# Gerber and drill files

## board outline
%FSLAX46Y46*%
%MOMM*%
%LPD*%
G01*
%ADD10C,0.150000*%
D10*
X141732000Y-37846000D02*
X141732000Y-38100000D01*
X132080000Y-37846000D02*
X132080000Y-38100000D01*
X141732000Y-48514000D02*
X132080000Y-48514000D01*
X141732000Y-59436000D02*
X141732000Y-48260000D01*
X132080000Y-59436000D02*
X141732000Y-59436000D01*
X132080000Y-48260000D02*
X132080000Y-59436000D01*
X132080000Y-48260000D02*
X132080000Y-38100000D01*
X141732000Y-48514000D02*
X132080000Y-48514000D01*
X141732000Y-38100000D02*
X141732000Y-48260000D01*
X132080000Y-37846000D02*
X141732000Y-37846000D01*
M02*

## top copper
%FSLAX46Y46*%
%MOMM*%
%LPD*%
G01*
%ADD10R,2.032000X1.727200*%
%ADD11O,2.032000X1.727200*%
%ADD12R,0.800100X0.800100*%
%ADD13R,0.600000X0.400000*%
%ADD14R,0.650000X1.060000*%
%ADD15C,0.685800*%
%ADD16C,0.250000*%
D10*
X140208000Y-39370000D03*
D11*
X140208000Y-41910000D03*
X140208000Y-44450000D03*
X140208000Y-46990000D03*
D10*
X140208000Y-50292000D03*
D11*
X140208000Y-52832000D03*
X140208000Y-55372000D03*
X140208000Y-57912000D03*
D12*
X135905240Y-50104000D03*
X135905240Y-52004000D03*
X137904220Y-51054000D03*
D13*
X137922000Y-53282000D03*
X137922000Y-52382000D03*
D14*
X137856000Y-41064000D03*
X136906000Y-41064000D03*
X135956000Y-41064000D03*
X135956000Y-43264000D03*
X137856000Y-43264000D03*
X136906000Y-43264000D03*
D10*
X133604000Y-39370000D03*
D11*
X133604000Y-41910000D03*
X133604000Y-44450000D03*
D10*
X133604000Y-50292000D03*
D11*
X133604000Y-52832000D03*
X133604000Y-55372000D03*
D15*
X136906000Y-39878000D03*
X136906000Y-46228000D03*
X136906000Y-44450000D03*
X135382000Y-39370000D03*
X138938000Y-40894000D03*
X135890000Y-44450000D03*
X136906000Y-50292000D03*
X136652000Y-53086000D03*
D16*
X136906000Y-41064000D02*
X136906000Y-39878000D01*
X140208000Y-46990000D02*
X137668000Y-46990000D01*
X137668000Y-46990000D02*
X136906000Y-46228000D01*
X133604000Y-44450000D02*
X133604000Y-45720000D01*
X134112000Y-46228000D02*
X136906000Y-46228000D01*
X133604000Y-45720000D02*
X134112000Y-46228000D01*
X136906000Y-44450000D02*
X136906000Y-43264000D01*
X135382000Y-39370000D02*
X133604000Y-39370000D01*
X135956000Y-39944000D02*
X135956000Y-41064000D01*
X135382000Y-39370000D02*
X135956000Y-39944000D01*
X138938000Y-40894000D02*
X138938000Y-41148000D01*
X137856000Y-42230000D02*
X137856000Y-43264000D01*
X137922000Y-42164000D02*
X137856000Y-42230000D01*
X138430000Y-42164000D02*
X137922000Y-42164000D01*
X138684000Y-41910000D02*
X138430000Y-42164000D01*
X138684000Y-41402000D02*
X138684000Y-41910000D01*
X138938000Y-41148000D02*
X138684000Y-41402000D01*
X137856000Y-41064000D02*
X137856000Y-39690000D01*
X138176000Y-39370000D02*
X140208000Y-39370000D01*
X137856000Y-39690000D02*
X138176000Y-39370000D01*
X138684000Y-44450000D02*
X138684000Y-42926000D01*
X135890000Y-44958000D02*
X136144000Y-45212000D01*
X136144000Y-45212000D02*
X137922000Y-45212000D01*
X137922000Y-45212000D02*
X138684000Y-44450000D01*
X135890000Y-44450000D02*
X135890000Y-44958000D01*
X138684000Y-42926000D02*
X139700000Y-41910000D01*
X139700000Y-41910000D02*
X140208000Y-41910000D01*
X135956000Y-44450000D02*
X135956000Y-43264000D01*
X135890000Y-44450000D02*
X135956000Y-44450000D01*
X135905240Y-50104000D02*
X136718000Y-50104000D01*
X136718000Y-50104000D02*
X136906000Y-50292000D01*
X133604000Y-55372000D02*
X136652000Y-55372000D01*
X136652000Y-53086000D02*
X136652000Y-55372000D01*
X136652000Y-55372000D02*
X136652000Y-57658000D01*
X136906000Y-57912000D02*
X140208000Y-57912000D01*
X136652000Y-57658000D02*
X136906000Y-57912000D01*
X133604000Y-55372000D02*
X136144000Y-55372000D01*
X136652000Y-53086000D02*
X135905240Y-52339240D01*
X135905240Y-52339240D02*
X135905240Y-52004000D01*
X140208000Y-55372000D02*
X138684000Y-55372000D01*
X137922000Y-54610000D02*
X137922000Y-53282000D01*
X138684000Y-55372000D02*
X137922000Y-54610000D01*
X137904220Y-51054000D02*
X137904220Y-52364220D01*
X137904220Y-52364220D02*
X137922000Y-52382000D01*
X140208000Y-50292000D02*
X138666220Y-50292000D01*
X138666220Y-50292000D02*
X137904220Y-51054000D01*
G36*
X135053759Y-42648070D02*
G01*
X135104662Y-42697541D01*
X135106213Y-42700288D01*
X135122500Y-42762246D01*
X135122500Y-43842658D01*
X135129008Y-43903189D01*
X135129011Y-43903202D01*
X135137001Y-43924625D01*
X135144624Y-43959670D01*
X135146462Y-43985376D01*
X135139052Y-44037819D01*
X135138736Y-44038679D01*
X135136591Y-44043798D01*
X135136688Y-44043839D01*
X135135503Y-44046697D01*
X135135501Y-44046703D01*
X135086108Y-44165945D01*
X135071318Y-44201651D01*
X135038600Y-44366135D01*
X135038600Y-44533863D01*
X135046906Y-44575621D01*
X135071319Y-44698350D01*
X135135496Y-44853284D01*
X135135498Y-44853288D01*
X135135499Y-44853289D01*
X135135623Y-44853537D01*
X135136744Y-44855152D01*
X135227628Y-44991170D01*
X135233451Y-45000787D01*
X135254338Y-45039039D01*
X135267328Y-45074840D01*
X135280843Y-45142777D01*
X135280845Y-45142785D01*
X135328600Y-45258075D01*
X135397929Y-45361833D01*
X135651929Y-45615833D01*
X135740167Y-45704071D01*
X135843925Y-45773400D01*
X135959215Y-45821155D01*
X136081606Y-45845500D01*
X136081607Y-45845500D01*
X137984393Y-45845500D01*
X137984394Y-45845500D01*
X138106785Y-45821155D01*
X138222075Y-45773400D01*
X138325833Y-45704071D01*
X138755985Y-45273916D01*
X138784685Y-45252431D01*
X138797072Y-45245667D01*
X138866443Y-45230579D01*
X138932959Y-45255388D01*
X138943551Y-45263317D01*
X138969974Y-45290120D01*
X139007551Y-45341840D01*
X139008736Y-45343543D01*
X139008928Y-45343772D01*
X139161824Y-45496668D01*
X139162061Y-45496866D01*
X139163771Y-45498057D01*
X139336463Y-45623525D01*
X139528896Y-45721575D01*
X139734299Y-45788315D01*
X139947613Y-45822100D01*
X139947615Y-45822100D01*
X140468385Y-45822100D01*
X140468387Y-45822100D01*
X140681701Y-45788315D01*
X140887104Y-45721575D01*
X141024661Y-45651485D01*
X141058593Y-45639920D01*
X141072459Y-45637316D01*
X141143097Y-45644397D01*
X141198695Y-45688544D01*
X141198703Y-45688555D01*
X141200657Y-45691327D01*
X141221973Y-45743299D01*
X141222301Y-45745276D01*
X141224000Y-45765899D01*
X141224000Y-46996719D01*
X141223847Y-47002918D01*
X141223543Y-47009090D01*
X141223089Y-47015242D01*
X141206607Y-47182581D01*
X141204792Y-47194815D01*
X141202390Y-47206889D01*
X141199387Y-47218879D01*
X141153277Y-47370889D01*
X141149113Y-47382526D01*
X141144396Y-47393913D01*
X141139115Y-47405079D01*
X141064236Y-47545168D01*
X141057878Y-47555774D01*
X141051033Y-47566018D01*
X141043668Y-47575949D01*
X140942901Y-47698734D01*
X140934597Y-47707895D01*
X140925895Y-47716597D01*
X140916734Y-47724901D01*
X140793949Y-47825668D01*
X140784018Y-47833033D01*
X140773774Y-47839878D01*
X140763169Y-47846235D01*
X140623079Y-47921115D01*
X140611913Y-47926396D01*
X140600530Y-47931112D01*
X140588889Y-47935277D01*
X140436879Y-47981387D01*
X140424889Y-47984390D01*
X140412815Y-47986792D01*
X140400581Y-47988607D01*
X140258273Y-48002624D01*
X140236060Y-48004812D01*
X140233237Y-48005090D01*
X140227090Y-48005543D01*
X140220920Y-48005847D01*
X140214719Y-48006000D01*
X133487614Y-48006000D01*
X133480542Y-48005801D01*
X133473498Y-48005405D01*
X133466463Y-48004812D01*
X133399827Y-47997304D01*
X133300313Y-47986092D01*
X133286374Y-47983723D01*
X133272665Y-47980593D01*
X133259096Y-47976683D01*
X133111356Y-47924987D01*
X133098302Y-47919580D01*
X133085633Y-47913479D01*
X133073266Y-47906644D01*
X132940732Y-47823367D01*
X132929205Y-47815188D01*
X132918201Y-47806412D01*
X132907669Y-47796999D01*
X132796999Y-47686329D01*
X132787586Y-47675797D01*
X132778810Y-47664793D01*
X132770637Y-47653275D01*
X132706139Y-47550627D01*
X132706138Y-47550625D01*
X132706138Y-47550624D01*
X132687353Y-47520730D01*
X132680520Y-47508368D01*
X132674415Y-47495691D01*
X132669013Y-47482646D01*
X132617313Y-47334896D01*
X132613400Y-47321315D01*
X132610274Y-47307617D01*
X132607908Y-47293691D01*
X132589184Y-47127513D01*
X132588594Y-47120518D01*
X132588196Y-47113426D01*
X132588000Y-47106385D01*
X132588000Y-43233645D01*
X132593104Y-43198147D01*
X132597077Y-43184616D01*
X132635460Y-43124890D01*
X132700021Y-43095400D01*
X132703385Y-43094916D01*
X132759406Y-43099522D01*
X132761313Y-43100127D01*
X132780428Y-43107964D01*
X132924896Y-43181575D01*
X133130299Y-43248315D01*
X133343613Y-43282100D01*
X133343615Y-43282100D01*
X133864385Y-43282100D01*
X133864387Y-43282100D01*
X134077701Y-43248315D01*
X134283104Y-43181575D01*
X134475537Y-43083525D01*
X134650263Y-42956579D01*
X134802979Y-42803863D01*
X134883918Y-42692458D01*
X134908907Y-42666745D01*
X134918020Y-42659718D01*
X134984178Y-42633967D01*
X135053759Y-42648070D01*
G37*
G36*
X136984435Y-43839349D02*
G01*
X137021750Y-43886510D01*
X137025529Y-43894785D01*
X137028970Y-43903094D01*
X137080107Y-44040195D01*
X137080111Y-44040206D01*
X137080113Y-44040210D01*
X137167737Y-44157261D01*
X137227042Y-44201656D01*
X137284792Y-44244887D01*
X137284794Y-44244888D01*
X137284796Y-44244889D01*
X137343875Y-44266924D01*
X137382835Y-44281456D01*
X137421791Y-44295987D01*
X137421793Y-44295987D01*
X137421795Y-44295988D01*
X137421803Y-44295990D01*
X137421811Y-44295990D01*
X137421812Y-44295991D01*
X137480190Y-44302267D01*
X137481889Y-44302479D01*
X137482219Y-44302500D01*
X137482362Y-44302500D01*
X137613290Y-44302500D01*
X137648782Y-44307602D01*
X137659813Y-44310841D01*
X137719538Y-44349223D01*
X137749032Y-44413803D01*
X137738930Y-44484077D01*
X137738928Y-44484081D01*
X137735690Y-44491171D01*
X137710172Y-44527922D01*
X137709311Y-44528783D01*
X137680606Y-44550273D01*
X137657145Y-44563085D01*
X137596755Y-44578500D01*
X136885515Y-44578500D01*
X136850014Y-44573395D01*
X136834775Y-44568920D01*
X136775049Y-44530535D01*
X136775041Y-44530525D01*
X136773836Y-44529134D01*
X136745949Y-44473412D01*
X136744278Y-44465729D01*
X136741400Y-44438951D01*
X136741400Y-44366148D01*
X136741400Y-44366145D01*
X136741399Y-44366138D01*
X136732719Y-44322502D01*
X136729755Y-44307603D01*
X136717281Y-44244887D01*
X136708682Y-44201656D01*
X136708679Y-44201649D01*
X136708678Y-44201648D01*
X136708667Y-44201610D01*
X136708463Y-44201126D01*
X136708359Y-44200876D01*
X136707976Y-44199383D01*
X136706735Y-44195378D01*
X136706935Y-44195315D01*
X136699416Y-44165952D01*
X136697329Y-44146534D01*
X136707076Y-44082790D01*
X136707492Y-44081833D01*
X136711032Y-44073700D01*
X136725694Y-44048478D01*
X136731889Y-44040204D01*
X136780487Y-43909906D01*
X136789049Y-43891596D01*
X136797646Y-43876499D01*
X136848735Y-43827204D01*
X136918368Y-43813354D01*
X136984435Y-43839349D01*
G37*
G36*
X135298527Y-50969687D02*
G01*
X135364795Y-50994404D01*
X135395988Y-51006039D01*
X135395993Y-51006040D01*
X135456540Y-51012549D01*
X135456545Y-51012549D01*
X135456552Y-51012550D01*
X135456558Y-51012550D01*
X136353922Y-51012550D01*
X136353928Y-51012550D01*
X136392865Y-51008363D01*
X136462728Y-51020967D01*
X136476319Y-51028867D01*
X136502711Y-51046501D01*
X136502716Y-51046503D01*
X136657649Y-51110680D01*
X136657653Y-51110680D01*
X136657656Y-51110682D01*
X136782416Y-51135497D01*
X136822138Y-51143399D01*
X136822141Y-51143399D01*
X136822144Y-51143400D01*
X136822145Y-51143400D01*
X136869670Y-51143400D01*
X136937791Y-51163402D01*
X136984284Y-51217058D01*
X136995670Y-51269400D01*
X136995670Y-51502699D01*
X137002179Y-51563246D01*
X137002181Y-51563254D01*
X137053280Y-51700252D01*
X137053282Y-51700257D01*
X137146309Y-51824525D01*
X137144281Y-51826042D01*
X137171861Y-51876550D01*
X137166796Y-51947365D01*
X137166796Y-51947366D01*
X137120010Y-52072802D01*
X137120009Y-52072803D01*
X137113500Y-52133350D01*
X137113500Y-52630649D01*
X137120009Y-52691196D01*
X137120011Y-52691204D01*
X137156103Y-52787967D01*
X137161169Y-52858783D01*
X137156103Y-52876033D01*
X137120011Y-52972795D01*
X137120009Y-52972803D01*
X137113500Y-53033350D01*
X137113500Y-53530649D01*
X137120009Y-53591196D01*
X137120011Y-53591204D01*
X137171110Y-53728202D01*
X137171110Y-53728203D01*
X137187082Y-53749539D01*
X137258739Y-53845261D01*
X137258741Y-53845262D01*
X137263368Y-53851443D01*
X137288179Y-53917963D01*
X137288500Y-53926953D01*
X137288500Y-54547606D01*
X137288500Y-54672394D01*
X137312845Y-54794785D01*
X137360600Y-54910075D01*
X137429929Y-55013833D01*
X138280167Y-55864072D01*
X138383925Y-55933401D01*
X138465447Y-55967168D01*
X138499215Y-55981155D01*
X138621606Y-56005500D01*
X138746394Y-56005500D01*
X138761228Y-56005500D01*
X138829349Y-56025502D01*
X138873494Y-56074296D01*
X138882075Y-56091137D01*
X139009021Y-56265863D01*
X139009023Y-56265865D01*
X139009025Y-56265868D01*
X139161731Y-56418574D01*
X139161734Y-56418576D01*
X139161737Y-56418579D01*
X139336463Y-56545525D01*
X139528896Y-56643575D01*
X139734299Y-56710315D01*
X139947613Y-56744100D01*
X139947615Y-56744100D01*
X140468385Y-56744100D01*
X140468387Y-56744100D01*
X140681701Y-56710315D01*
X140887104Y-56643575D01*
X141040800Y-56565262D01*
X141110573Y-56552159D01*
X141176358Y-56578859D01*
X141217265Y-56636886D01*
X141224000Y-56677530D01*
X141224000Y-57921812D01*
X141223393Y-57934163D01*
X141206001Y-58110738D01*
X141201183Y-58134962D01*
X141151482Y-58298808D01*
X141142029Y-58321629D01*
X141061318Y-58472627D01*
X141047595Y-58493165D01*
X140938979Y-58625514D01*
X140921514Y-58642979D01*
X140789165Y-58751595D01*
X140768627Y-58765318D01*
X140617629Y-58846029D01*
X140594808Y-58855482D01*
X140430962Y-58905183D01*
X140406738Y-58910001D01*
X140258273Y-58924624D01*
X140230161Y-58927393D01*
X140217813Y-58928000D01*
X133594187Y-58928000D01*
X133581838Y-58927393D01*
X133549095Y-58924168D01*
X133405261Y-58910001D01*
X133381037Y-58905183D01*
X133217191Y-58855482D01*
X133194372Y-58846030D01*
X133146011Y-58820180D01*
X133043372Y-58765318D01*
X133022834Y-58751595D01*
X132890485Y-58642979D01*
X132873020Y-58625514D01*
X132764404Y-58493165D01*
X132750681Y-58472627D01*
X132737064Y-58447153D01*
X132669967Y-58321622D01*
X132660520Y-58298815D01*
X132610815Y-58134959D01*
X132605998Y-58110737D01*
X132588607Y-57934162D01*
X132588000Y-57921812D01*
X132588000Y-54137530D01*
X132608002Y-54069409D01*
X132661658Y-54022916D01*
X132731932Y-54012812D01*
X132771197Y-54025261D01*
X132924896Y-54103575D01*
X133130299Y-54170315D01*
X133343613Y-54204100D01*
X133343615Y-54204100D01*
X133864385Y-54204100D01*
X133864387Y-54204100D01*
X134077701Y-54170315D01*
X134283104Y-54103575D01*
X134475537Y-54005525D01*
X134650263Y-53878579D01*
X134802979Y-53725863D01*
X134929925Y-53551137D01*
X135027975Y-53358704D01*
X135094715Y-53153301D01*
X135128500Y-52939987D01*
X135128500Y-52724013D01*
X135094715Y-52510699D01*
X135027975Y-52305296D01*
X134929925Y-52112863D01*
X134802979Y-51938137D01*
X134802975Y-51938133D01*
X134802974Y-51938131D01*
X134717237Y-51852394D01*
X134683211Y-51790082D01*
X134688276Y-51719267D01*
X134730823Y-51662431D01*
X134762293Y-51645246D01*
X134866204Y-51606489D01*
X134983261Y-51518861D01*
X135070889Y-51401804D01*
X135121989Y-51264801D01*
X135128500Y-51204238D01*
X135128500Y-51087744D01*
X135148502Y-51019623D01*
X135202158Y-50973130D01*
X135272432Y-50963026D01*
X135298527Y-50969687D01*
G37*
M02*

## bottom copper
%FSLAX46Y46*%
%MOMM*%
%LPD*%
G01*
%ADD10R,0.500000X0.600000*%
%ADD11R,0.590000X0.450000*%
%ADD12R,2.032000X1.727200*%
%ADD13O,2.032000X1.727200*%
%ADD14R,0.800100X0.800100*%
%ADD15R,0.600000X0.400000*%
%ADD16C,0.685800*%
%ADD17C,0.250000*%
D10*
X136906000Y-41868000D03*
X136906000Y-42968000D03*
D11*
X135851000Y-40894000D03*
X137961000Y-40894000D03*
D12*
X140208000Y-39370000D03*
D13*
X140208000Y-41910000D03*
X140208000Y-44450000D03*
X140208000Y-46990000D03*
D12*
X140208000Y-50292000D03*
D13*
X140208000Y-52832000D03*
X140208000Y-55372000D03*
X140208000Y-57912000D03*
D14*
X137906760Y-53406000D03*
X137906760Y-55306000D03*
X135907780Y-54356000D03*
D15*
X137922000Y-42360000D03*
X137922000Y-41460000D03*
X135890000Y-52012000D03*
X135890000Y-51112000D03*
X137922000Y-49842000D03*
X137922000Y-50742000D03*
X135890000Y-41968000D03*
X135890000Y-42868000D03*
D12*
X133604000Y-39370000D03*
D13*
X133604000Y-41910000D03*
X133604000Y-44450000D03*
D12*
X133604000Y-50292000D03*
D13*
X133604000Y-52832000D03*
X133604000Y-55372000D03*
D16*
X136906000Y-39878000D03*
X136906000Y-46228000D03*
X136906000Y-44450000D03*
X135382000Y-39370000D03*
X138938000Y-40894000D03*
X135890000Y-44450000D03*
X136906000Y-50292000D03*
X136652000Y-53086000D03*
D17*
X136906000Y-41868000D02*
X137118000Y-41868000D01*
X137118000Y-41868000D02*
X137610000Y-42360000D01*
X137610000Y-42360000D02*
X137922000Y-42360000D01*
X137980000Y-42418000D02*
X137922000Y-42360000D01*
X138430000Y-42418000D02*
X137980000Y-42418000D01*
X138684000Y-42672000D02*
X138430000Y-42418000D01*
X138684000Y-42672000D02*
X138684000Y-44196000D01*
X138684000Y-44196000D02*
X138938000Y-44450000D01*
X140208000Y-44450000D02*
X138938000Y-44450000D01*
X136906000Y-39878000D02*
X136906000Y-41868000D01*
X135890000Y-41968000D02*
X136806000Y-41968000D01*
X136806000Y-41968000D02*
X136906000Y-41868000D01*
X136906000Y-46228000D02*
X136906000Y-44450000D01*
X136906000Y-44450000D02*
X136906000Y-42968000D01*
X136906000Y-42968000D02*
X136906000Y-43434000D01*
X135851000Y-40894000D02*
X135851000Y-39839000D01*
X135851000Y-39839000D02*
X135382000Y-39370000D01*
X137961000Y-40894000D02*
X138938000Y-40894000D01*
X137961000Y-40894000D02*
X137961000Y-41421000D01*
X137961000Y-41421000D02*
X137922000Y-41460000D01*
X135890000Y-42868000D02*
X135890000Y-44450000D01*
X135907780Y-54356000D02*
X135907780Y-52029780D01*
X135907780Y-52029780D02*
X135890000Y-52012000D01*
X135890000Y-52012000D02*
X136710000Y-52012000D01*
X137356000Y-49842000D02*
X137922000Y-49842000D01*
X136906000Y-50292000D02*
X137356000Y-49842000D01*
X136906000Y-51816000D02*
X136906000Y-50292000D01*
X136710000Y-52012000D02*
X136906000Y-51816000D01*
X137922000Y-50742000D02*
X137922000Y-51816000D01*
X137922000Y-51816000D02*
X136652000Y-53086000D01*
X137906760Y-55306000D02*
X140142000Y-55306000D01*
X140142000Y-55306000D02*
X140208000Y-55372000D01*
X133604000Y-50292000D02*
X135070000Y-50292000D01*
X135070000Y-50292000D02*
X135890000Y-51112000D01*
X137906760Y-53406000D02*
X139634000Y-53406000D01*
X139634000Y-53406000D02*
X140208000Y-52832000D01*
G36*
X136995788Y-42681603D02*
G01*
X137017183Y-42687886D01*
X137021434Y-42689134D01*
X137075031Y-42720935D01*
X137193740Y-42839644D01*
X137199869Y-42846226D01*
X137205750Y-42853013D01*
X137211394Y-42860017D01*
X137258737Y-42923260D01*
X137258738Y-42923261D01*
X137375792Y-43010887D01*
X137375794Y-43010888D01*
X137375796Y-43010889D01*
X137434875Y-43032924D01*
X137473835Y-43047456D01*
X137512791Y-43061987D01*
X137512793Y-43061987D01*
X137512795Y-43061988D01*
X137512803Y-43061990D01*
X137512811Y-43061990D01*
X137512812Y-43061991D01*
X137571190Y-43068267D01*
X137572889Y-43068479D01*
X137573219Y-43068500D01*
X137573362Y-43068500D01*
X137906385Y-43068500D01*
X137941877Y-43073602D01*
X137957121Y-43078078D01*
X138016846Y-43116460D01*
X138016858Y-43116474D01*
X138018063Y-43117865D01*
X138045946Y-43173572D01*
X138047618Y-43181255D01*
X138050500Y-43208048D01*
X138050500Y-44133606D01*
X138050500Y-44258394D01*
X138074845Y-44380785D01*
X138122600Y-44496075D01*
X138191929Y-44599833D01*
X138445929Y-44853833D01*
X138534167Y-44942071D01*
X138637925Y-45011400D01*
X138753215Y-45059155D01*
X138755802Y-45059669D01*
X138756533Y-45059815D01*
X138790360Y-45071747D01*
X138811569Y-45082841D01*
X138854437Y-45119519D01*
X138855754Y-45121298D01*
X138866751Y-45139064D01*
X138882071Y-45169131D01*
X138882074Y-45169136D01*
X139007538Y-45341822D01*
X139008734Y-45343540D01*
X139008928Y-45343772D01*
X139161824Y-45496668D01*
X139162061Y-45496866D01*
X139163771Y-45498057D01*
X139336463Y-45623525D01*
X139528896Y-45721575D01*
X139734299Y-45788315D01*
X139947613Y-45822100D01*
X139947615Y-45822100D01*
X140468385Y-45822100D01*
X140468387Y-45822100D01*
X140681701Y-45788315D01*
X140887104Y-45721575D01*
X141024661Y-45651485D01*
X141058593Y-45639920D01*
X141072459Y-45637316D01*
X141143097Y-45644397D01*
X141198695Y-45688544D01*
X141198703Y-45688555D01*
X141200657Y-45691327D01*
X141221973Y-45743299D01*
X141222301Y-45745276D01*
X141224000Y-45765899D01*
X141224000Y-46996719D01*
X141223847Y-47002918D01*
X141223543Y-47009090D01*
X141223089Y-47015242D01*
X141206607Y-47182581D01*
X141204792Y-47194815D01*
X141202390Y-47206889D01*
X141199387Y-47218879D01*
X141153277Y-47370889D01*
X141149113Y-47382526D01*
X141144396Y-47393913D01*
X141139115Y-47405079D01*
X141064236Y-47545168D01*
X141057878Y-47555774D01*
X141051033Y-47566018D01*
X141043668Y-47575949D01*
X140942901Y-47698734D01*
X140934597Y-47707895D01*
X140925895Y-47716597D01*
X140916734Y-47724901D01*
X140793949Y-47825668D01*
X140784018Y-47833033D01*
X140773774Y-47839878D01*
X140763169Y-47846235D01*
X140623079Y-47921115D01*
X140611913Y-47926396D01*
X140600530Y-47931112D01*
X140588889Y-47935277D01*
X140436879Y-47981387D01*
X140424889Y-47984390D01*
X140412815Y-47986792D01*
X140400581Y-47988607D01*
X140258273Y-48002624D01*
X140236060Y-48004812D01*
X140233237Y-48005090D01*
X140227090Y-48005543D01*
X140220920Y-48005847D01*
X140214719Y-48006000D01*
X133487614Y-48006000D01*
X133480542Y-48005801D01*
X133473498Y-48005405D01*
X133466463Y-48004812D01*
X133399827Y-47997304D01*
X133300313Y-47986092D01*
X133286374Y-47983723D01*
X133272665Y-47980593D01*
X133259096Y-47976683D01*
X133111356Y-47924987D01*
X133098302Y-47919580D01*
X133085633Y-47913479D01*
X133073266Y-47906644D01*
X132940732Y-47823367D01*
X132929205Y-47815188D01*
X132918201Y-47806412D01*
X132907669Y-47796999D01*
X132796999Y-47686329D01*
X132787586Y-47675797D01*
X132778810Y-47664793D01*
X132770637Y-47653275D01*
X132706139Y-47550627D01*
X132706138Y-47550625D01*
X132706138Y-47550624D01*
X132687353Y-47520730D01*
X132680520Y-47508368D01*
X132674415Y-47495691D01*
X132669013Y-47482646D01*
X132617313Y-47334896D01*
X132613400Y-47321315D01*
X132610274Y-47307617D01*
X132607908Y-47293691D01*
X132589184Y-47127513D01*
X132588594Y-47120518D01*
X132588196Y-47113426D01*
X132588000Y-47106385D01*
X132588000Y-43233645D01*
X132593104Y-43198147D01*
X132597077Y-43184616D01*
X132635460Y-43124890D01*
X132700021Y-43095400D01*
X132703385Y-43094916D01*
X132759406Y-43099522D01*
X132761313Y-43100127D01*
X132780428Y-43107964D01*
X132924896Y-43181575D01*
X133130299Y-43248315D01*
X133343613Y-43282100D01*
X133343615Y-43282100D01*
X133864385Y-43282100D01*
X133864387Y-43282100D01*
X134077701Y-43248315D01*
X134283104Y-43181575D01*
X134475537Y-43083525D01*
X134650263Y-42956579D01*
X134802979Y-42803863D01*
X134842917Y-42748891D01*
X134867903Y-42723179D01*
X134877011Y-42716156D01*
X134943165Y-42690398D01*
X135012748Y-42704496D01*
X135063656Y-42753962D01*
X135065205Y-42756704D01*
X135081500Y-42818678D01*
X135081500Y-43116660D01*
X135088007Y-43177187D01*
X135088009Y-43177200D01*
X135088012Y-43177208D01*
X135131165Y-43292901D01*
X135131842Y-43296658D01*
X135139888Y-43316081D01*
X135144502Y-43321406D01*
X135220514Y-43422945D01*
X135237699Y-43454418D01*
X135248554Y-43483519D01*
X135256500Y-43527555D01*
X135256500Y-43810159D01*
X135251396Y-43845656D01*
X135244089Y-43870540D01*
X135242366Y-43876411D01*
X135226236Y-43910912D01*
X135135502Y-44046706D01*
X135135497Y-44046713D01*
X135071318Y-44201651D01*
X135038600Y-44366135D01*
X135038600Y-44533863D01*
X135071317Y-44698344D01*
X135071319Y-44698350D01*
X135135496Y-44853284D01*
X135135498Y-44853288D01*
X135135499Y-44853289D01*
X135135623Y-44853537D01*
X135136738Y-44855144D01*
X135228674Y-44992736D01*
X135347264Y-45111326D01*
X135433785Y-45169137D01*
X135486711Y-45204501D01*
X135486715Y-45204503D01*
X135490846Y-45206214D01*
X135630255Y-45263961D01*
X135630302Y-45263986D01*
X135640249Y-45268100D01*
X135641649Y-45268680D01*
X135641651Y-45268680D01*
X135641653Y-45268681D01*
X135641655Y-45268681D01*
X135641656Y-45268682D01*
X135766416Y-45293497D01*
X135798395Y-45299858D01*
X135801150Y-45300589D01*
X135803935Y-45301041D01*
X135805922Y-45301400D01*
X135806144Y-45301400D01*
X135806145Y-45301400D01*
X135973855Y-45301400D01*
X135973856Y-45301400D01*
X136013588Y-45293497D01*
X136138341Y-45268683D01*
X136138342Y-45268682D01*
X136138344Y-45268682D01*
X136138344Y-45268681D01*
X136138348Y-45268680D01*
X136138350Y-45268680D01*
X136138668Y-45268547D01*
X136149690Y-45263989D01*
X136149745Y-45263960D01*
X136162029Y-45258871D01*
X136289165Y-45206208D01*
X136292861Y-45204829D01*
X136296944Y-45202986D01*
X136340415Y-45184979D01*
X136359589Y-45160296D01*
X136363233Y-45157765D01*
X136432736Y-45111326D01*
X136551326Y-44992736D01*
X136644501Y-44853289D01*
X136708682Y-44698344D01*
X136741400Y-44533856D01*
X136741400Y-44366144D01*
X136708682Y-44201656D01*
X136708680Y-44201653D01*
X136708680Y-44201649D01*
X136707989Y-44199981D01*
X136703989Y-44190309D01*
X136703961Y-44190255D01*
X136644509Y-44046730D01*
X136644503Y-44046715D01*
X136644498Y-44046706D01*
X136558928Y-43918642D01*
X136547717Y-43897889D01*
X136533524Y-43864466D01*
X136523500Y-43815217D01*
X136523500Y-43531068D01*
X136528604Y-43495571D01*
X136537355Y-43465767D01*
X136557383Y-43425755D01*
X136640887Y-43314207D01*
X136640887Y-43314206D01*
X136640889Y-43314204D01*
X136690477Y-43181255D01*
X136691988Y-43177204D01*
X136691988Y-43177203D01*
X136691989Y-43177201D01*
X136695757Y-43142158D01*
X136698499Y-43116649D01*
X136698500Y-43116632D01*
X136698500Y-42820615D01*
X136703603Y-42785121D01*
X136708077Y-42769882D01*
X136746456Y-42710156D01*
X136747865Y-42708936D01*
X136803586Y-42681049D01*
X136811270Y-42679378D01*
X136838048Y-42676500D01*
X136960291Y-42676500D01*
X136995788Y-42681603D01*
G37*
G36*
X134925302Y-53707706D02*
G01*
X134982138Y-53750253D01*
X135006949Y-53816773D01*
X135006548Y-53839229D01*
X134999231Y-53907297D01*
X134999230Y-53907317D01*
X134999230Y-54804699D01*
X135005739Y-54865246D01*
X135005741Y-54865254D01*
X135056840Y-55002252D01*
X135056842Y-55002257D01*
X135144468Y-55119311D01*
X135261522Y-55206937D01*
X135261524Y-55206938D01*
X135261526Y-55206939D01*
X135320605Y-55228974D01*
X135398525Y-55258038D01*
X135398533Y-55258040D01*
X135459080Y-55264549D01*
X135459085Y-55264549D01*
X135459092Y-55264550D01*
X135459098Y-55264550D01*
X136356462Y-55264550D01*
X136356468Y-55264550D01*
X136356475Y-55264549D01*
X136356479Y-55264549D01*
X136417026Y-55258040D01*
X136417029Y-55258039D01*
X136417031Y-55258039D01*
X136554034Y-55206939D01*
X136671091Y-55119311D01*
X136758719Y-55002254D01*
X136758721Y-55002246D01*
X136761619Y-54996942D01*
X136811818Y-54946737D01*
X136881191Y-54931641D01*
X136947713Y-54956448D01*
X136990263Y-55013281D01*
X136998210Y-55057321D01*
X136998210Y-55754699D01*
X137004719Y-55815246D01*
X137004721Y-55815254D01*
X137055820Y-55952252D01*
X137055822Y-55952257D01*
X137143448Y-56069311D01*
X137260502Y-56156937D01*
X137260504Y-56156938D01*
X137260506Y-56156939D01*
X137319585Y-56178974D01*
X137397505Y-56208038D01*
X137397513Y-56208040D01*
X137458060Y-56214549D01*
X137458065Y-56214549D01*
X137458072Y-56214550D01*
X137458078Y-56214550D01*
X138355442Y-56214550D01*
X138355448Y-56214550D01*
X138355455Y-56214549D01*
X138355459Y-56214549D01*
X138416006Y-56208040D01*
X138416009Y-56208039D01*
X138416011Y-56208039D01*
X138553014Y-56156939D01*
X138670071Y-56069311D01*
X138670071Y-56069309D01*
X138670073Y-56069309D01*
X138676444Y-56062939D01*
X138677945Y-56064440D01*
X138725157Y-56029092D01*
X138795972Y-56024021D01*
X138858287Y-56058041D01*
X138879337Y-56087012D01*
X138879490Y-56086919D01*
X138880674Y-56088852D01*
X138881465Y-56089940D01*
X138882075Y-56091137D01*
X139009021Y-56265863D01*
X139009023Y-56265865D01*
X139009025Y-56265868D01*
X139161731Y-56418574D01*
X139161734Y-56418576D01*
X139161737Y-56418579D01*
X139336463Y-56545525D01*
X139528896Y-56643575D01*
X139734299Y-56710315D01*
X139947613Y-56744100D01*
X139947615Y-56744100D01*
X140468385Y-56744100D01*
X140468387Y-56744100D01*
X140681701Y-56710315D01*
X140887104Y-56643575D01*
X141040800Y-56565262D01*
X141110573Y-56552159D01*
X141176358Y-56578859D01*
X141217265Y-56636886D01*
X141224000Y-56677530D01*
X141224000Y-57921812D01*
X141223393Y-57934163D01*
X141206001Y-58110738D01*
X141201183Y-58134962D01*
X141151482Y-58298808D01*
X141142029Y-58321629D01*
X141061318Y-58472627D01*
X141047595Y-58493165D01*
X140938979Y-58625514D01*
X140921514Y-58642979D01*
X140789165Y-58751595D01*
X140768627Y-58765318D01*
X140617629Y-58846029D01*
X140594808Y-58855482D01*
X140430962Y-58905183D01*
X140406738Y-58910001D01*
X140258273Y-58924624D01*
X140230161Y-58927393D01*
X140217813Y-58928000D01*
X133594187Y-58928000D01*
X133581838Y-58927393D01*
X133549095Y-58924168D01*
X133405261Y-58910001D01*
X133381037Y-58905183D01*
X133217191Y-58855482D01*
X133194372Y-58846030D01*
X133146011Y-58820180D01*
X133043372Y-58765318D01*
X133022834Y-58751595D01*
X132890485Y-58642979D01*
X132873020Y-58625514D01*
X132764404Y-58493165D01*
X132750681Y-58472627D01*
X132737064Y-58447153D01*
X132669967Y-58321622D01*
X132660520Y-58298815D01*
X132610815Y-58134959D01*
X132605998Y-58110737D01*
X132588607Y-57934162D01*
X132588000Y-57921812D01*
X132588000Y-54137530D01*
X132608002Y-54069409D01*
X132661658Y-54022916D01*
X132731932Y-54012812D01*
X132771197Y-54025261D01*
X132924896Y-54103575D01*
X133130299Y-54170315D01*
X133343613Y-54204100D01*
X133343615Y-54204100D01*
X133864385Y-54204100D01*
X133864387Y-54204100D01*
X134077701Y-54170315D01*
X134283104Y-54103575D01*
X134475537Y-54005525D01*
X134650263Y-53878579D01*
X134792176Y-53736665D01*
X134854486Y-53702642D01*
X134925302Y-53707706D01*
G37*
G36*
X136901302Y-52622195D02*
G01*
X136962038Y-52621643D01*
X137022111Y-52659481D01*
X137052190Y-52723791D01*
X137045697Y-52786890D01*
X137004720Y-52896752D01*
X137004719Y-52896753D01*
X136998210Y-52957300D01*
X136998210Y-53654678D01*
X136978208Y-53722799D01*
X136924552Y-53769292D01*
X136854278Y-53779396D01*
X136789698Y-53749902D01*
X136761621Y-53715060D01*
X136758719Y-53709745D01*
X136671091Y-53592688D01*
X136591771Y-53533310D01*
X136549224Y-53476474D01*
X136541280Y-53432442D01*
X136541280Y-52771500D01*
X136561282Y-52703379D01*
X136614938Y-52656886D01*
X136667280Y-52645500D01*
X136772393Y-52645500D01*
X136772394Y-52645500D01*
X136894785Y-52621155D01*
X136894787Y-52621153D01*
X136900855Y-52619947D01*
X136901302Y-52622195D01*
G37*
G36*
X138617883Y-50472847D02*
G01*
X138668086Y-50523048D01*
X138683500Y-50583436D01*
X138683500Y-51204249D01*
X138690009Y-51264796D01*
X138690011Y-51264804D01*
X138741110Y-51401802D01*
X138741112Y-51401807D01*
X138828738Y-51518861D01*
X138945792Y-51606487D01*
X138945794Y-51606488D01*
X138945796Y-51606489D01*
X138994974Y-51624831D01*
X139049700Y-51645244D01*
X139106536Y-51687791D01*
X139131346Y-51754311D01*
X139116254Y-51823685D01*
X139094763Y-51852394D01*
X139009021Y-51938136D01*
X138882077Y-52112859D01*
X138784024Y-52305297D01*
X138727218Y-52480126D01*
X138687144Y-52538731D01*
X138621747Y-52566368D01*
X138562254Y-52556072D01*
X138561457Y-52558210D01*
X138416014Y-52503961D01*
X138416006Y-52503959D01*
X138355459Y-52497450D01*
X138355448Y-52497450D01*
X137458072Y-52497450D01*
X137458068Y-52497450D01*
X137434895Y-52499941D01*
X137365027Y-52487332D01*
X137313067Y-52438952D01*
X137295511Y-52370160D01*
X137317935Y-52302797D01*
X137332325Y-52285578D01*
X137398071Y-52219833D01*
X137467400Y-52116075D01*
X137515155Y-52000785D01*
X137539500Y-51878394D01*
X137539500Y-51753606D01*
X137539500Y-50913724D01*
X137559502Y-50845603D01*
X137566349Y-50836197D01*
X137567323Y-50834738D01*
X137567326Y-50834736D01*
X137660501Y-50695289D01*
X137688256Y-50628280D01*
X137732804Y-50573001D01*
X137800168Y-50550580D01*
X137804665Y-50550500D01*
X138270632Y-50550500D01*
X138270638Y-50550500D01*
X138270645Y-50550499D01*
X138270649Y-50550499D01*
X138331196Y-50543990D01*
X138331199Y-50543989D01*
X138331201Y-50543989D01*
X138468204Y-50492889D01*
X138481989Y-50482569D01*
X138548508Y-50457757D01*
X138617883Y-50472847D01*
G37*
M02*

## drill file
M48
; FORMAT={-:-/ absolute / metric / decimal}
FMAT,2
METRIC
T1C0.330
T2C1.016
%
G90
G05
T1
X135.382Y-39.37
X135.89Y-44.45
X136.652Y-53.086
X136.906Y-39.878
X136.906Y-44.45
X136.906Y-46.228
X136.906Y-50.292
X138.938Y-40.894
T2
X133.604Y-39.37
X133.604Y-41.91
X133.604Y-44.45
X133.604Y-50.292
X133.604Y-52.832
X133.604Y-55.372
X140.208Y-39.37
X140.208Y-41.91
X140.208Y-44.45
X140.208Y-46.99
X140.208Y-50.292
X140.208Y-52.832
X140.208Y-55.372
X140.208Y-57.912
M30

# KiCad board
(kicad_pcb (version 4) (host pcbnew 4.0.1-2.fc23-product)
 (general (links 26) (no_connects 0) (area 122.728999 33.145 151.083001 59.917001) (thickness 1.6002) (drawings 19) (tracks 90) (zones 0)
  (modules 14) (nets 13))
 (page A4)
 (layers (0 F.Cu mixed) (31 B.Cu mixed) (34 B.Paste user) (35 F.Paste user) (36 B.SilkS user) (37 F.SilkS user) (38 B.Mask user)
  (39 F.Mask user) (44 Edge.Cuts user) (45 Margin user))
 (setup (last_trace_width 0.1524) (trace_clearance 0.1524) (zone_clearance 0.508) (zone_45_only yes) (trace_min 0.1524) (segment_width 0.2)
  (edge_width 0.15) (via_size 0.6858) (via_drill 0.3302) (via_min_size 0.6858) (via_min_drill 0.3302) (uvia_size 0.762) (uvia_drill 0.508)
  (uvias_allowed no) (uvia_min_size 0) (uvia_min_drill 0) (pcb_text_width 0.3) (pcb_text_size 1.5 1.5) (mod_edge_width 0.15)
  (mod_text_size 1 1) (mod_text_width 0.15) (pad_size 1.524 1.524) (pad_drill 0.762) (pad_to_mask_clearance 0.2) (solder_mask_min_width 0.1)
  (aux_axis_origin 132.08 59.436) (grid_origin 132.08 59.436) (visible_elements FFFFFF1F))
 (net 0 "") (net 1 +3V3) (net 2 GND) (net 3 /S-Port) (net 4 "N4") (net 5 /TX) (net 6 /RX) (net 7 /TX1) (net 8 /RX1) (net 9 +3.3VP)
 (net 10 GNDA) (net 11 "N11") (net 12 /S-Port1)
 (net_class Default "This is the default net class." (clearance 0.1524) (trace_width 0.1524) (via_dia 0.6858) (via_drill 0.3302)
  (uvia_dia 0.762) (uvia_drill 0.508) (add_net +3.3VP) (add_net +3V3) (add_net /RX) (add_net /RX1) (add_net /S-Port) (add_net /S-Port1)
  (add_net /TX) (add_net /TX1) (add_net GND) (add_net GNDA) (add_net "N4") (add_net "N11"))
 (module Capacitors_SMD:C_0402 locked (layer B.Cu) (at 136.906 42.418 270)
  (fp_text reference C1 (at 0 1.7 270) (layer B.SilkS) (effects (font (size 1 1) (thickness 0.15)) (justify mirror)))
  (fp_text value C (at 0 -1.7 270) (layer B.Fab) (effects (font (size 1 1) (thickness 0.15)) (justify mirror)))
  (pad 1 smd rect (at -0.55 0 270) (size 0.6 0.5) (layers B.Cu B.Paste B.Mask) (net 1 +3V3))
  (pad 2 smd rect (at 0.55 0 270) (size 0.6 0.5) (layers B.Cu B.Paste B.Mask) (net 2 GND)))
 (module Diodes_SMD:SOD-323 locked (layer B.Cu) (at 136.906 40.894)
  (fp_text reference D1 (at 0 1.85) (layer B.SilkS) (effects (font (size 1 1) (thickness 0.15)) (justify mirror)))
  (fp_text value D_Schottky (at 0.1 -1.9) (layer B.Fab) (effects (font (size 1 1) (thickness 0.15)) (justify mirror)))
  (pad 1 smd rect (at -1.055 0) (size 0.59 0.45) (layers B.Cu B.Paste B.Mask) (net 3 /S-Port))
  (pad 2 smd rect (at 1.055 0) (size 0.59 0.45) (layers B.Cu B.Paste B.Mask) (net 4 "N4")))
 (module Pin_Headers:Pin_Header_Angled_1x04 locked (layer F.Cu) (at 140.208 39.37)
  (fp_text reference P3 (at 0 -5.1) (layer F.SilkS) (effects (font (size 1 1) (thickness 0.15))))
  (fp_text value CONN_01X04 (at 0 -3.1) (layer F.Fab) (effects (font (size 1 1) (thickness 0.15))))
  (pad 1 thru_hole rect (at 0 0) (size 2.032 1.7272) (drill 1.016) (layers *.Cu *.Mask F.SilkS) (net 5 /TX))
  (pad 2 thru_hole oval (at 0 2.54) (size 2.032 1.7272) (drill 1.016) (layers *.Cu *.Mask F.SilkS) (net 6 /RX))
  (pad 3 thru_hole oval (at 0 5.08) (size 2.032 1.7272) (drill 1.016) (layers *.Cu *.Mask F.SilkS) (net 1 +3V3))
  (pad 4 thru_hole oval (at 0 7.62) (size 2.032 1.7272) (drill 1.016) (layers *.Cu *.Mask F.SilkS) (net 2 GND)))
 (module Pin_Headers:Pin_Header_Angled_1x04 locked (layer F.Cu) (at 140.208 50.292)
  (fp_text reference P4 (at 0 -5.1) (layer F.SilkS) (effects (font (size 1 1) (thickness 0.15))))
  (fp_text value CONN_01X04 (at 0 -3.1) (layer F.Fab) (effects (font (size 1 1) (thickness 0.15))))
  (pad 1 thru_hole rect (at 0 0) (size 2.032 1.7272) (drill 1.016) (layers *.Cu *.Mask F.SilkS) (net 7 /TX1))
  (pad 2 thru_hole oval (at 0 2.54) (size 2.032 1.7272) (drill 1.016) (layers *.Cu *.Mask F.SilkS) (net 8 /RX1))
  (pad 3 thru_hole oval (at 0 5.08) (size 2.032 1.7272) (drill 1.016) (layers *.Cu *.Mask F.SilkS) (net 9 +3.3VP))
  (pad 4 thru_hole oval (at 0 7.62) (size 2.032 1.7272) (drill 1.016) (layers *.Cu *.Mask F.SilkS) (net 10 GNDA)))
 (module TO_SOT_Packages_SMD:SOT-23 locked (layer B.Cu) (at 136.906 54.356 270)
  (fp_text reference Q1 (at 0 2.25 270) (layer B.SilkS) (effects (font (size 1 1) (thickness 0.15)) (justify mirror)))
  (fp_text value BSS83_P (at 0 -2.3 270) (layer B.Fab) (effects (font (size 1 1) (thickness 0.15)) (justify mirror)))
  (pad 1 smd rect (at -0.95 -1.00076 270) (size 0.8001 0.8001) (layers B.Cu B.Paste B.Mask) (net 8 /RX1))
  (pad 2 smd rect (at 0.95 -1.00076 270) (size 0.8001 0.8001) (layers B.Cu B.Paste B.Mask) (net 9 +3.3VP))
  (pad 3 smd rect (at 0 0.99822 270) (size 0.8001 0.8001) (layers B.Cu B.Paste B.Mask) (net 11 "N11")))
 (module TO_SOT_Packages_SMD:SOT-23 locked (layer F.Cu) (at 136.906 51.054 270)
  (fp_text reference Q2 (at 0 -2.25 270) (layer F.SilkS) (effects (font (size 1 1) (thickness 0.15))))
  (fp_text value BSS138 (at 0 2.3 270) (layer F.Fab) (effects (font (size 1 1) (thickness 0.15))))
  (pad 1 smd rect (at -0.95 1.00076 270) (size 0.8001 0.8001) (layers F.Cu F.Paste F.Mask) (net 11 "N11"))
  (pad 2 smd rect (at 0.95 1.00076 270) (size 0.8001 0.8001) (layers F.Cu F.Paste F.Mask) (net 10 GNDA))
  (pad 3 smd rect (at 0 -0.99822 270) (size 0.8001 0.8001) (layers F.Cu F.Paste F.Mask) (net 7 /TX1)))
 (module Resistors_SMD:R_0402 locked (layer B.Cu) (at 137.922 41.91 90)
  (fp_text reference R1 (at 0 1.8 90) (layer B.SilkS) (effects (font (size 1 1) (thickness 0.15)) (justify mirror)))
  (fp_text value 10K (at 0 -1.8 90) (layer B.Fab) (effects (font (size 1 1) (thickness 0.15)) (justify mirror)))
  (pad 1 smd rect (at -0.45 0 90) (size 0.4 0.6) (layers B.Cu B.Paste B.Mask) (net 1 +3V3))
  (pad 2 smd rect (at 0.45 0 90) (size 0.4 0.6) (layers B.Cu B.Paste B.Mask) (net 4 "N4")))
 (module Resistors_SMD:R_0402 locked (layer B.Cu) (at 135.89 51.562 90)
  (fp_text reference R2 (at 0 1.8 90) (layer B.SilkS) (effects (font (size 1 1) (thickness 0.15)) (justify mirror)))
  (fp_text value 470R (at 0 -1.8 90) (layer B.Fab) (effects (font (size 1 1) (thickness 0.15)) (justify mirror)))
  (pad 1 smd rect (at -0.45 0 90) (size 0.4 0.6) (layers B.Cu B.Paste B.Mask) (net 11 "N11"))
  (pad 2 smd rect (at 0.45 0 90) (size 0.4 0.6) (layers B.Cu B.Paste B.Mask) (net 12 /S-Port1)))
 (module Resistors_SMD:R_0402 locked (layer B.Cu) (at 137.922 50.292 270)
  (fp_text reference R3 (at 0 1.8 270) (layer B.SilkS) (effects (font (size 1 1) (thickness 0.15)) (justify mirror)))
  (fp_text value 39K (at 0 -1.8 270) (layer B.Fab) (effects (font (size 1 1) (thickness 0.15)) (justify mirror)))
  (pad 1 smd rect (at -0.45 0 270) (size 0.4 0.6) (layers B.Cu B.Paste B.Mask) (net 11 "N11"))
  (pad 2 smd rect (at 0.45 0 270) (size 0.4 0.6) (layers B.Cu B.Paste B.Mask) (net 10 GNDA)))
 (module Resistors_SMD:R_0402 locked (layer F.Cu) (at 137.922 52.832 90)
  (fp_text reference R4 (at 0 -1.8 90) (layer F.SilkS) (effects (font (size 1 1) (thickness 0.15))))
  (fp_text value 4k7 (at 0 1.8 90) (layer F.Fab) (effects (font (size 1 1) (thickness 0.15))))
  (pad 1 smd rect (at -0.45 0 90) (size 0.4 0.6) (layers F.Cu F.Paste F.Mask) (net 9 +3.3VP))
  (pad 2 smd rect (at 0.45 0 90) (size 0.4 0.6) (layers F.Cu F.Paste F.Mask) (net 7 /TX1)))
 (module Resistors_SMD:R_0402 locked (layer B.Cu) (at 135.89 42.418 270)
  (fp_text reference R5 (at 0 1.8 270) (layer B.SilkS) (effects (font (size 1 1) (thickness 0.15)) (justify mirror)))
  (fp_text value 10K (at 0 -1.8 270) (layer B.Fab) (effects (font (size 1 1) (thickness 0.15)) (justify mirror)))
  (pad 1 smd rect (at -0.45 0 270) (size 0.4 0.6) (layers B.Cu B.Paste B.Mask) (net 1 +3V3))
  (pad 2 smd rect (at 0.45 0 270) (size 0.4 0.6) (layers B.Cu B.Paste B.Mask) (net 6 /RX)))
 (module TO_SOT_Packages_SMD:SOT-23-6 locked (layer F.Cu) (at 136.906 42.164 270)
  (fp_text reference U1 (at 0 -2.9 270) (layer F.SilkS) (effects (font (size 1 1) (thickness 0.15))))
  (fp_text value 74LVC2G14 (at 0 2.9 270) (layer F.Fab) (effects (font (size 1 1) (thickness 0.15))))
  (pad 1 smd rect (at -1.1 -0.95 270) (size 1.06 0.65) (layers F.Cu F.Paste F.Mask) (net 5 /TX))
  (pad 2 smd rect (at -1.1 0 270) (size 1.06 0.65) (layers F.Cu F.Paste F.Mask) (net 1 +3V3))
  (pad 3 smd rect (at -1.1 0.95 270) (size 1.06 0.65) (layers F.Cu F.Paste F.Mask) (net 3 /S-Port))
  (pad 4 smd rect (at 1.1 0.95 270) (size 1.06 0.65) (layers F.Cu F.Paste F.Mask) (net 6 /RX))
  (pad 6 smd rect (at 1.1 -0.95 270) (size 1.06 0.65) (layers F.Cu F.Paste F.Mask) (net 4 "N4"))
  (pad 5 smd rect (at 1.1 0 270) (size 1.06 0.65) (layers F.Cu F.Paste F.Mask) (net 2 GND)))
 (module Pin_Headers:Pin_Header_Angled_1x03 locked (layer B.Cu) (at 133.604 39.37 180)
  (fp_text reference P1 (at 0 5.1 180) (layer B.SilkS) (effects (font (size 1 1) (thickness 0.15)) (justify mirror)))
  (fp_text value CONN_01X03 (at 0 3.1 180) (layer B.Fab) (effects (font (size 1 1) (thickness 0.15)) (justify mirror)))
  (pad 1 thru_hole rect (at 0 0 180) (size 2.032 1.7272) (drill 1.016) (layers *.Cu *.Mask B.SilkS) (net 3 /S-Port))
  (pad 2 thru_hole oval (at 0 -2.54 180) (size 2.032 1.7272) (drill 1.016) (layers *.Cu *.Mask B.SilkS))
  (pad 3 thru_hole oval (at 0 -5.08 180) (size 2.032 1.7272) (drill 1.016) (layers *.Cu *.Mask B.SilkS) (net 2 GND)))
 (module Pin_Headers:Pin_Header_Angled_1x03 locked (layer B.Cu) (at 133.604 50.292 180)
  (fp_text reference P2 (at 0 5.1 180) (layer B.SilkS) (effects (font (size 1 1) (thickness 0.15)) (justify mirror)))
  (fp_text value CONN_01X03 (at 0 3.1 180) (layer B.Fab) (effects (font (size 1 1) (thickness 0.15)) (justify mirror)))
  (pad 1 thru_hole rect (at 0 0 180) (size 2.032 1.7272) (drill 1.016) (layers *.Cu *.Mask B.SilkS) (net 12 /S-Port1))
  (pad 2 thru_hole oval (at 0 -2.54 180) (size 2.032 1.7272) (drill 1.016) (layers *.Cu *.Mask B.SilkS))
  (pad 3 thru_hole oval (at 0 -5.08 180) (size 2.032 1.7272) (drill 1.016) (layers *.Cu *.Mask B.SilkS) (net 10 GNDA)))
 (gr_line (start 141.732 37.846) (end 141.732 38.1) (angle 90) (layer Edge.Cuts) (width 0.15))
 (gr_line (start 132.08 37.846) (end 132.08 38.1) (angle 90) (layer Edge.Cuts) (width 0.15))
 (gr_line (start 141.732 48.514) (end 132.08 48.514) (angle 90) (layer Edge.Cuts) (width 0.15))
 (gr_line (start 141.732 59.436) (end 141.732 48.26) (angle 90) (layer Edge.Cuts) (width 0.15))
 (gr_line (start 132.08 59.436) (end 141.732 59.436) (angle 90) (layer Edge.Cuts) (width 0.15))
 (gr_line (start 132.08 48.26) (end 132.08 59.436) (angle 90) (layer Edge.Cuts) (width 0.15))
 (gr_line (start 132.08 48.26) (end 132.08 38.1) (angle 90) (layer Edge.Cuts) (width 0.15))
 (gr_line (start 141.732 48.514) (end 132.08 48.514) (angle 90) (layer Edge.Cuts) (width 0.15))
 (gr_line (start 141.732 38.1) (end 141.732 48.26) (angle 90) (layer Edge.Cuts) (width 0.15))
 (gr_line (start 132.08 37.846) (end 141.732 37.846) (angle 90) (layer Edge.Cuts) (width 0.15))
 (segment (start 136.906 41.868) (end 137.118 41.868) (width 0.25) (layer B.Cu) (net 1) (status 30))
 (segment (start 137.118 41.868) (end 137.61 42.36) (width 0.25) (layer B.Cu) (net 1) (status 10))
 (segment (start 137.61 42.36) (end 137.922 42.36) (width 0.25) (layer B.Cu) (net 1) (status 20))
 (segment (start 137.98 42.418) (end 137.922 42.36) (width 0.25) (layer B.Cu) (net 1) (status 30))
 (segment (start 138.43 42.418) (end 137.98 42.418) (width 0.25) (layer B.Cu) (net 1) (status 20))
 (segment (start 138.684 42.672) (end 138.43 42.418) (width 0.25) (layer B.Cu) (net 1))
 (segment (start 138.684 42.672) (end 138.684 44.196) (width 0.25) (layer B.Cu) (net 1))
 (segment (start 138.684 44.196) (end 138.938 44.45) (width 0.25) (layer B.Cu) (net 1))
 (segment (start 140.208 44.45) (end 138.938 44.45) (width 0.25) (layer B.Cu) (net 1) (status 10))
 (segment (start 136.906 41.064) (end 136.906 39.878) (width 0.25) (layer F.Cu) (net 1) (status 10))
 (segment (start 136.906 39.878) (end 136.906 41.868) (width 0.25) (layer B.Cu) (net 1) (status 20))
 (via (at 136.906 39.878) (size 0.6858) (drill 0.3302) (layers F.Cu B.Cu) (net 1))
 (segment (start 135.89 41.968) (end 136.806 41.968) (width 0.25) (layer B.Cu) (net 1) (status 30))
 (segment (start 136.806 41.968) (end 136.906 41.868) (width 0.25) (layer B.Cu) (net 1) (status 30))
 (segment (start 140.208 46.99) (end 137.668 46.99) (width 0.25) (layer F.Cu) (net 2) (status 10))
 (segment (start 137.668 46.99) (end 136.906 46.228) (width 0.25) (layer F.Cu) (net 2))
 (segment (start 133.604 44.45) (end 133.604 45.72) (width 0.25) (layer F.Cu) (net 2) (status 10))
 (segment (start 134.112 46.228) (end 136.906 46.228) (width 0.25) (layer F.Cu) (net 2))
 (segment (start 133.604 45.72) (end 134.112 46.228) (width 0.25) (layer F.Cu) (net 2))
 (segment (start 136.906 46.228) (end 136.906 44.45) (width 0.25) (layer B.Cu) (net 2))
 (via (at 136.906 46.228) (size 0.6858) (drill 0.3302) (layers F.Cu B.Cu) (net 2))
 (via (at 136.906 44.45) (size 0.6858) (drill 0.3302) (layers F.Cu B.Cu) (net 2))
 (segment (start 136.906 44.45) (end 136.906 42.968) (width 0.25) (layer B.Cu) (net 2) (status 20))
 (segment (start 136.906 42.968) (end 136.906 43.434) (width 0.25) (layer B.Cu) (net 2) (status 10))
 (segment (start 136.906 44.45) (end 136.906 43.264) (width 0.25) (layer F.Cu) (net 2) (status 20))
 (segment (start 135.851 40.894) (end 135.851 39.839) (width 0.25) (layer B.Cu) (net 3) (status 10))
 (via (at 135.382 39.37) (size 0.6858) (drill 0.3302) (layers F.Cu B.Cu) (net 3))
 (segment (start 135.851 39.839) (end 135.382 39.37) (width 0.25) (layer B.Cu) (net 3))
 (segment (start 135.382 39.37) (end 133.604 39.37) (width 0.25) (layer F.Cu) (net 3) (status 20))
 (segment (start 135.956 39.944) (end 135.956 41.064) (width 0.25) (layer F.Cu) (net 3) (status 20))
 (segment (start 135.382 39.37) (end 135.956 39.944) (width 0.25) (layer F.Cu) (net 3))
 (segment (start 138.938 40.894) (end 138.938 41.148) (width 0.25) (layer F.Cu) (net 4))
 (via (at 138.938 40.894) (size 0.6858) (drill 0.3302) (layers F.Cu B.Cu) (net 4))
 (segment (start 137.961 40.894) (end 138.938 40.894) (width 0.25) (layer B.Cu) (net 4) (status 10))
 (segment (start 137.856 42.23) (end 137.856 43.264) (width 0.25) (layer F.Cu) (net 4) (status 20))
 (segment (start 137.922 42.164) (end 137.856 42.23) (width 0.25) (layer F.Cu) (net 4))
 (segment (start 138.43 42.164) (end 137.922 42.164) (width 0.25) (layer F.Cu) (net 4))
 (segment (start 138.684 41.91) (end 138.43 42.164) (width 0.25) (layer F.Cu) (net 4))
 (segment (start 138.684 41.402) (end 138.684 41.91) (width 0.25) (layer F.Cu) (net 4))
 (segment (start 138.938 41.148) (end 138.684 41.402) (width 0.25) (layer F.Cu) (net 4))
 (segment (start 137.961 40.894) (end 137.961 41.421) (width 0.25) (layer B.Cu) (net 4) (status 30))
 (segment (start 137.961 41.421) (end 137.922 41.46) (width 0.25) (layer B.Cu) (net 4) (status 30))
 (segment (start 137.856 41.064) (end 137.856 39.69) (width 0.25) (layer F.Cu) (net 5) (status 10))
 (segment (start 138.176 39.37) (end 140.208 39.37) (width 0.25) (layer F.Cu) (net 5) (status 20))
 (segment (start 137.856 39.69) (end 138.176 39.37) (width 0.25) (layer F.Cu) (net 5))
 (segment (start 138.684 44.45) (end 138.684 42.926) (width 0.25) (layer F.Cu) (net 6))
 (segment (start 135.89 44.958) (end 136.144 45.212) (width 0.25) (layer F.Cu) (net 6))
 (segment (start 136.144 45.212) (end 137.922 45.212) (width 0.25) (layer F.Cu) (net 6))
 (segment (start 137.922 45.212) (end 138.684 44.45) (width 0.25) (layer F.Cu) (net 6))
 (segment (start 135.89 44.45) (end 135.89 44.958) (width 0.25) (layer F.Cu) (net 6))
 (segment (start 138.684 42.926) (end 139.7 41.91) (width 0.25) (layer F.Cu) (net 6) (status 20))
 (segment (start 139.7 41.91) (end 140.208 41.91) (width 0.25) (layer F.Cu) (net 6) (status 30))
 (segment (start 135.89 42.868) (end 135.89 44.45) (width 0.25) (layer B.Cu) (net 6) (status 10))
 (segment (start 135.956 44.45) (end 135.956 43.264) (width 0.25) (layer F.Cu) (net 6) (status 20))
 (segment (start 135.89 44.45) (end 135.956 44.45) (width 0.25) (layer F.Cu) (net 6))
 (via (at 135.89 44.45) (size 0.6858) (drill 0.3302) (layers F.Cu B.Cu) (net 6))
 (segment (start 135.90524 50.104) (end 136.718 50.104) (width 0.25) (layer F.Cu) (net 11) (status 10))
 (via (at 136.906 50.292) (size 0.6858) (drill 0.3302) (layers F.Cu B.Cu) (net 11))
 (segment (start 136.718 50.104) (end 136.906 50.292) (width 0.25) (layer F.Cu) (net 11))
 (segment (start 135.90778 54.356) (end 135.90778 52.02978) (width 0.25) (layer B.Cu) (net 11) (status 30))
 (segment (start 135.90778 52.02978) (end 135.89 52.012) (width 0.25) (layer B.Cu) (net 11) (status 30))
 (segment (start 135.89 52.012) (end 136.71 52.012) (width 0.25) (layer B.Cu) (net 11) (status 10))
 (segment (start 137.356 49.842) (end 137.922 49.842) (width 0.25) (layer B.Cu) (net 11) (status 20))
 (segment (start 136.906 50.292) (end 137.356 49.842) (width 0.25) (layer B.Cu) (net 11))
 (segment (start 136.906 51.816) (end 136.906 50.292) (width 0.25) (layer B.Cu) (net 11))
 (segment (start 136.71 52.012) (end 136.906 51.816) (width 0.25) (layer B.Cu) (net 11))
 (segment (start 133.604 55.372) (end 136.652 55.372) (width 0.25) (layer F.Cu) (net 10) (status 10))
 (segment (start 136.652 53.086) (end 136.652 55.372) (width 0.25) (layer F.Cu) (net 10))
 (segment (start 136.652 55.372) (end 136.652 57.658) (width 0.25) (layer F.Cu) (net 10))
 (segment (start 136.906 57.912) (end 140.208 57.912) (width 0.25) (layer F.Cu) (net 10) (status 20))
 (segment (start 136.652 57.658) (end 136.906 57.912) (width 0.25) (layer F.Cu) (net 10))
 (segment (start 133.604 55.372) (end 136.144 55.372) (width 0.25) (layer F.Cu) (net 10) (status 10))
 (via (at 136.652 53.086) (size 0.6858) (drill 0.3302) (layers F.Cu B.Cu) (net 10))
 (segment (start 137.922 50.742) (end 137.922 51.816) (width 0.25) (layer B.Cu) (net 10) (status 10))
 (segment (start 137.922 51.816) (end 136.652 53.086) (width 0.25) (layer B.Cu) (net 10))
 (segment (start 136.652 53.086) (end 135.90524 52.33924) (width 0.25) (layer F.Cu) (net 10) (status 20))
 (segment (start 135.90524 52.33924) (end 135.90524 52.004) (width 0.25) (layer F.Cu) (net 10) (status 30))
 (segment (start 140.208 55.372) (end 138.684 55.372) (width 0.25) (layer F.Cu) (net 9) (status 10))
 (segment (start 137.922 54.61) (end 137.922 53.282) (width 0.25) (layer F.Cu) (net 9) (status 20))
 (segment (start 138.684 55.372) (end 137.922 54.61) (width 0.25) (layer F.Cu) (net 9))
 (segment (start 137.90676 55.306) (end 140.142 55.306) (width 0.25) (layer B.Cu) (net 9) (status 30))
 (segment (start 140.142 55.306) (end 140.208 55.372) (width 0.25) (layer B.Cu) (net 9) (status 30))
 (segment (start 133.604 50.292) (end 135.07 50.292) (width 0.25) (layer B.Cu) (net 12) (status 10))
 (segment (start 135.07 50.292) (end 135.89 51.112) (width 0.25) (layer B.Cu) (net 12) (status 20))
 (segment (start 137.90422 51.054) (end 137.90422 52.36422) (width 0.25) (layer F.Cu) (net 7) (status 30))
 (segment (start 137.90422 52.36422) (end 137.922 52.382) (width 0.25) (layer F.Cu) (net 7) (status 30))
 (segment (start 140.208 50.292) (end 138.66622 50.292) (width 0.25) (layer F.Cu) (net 7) (status 10))
 (segment (start 138.66622 50.292) (end 137.90422 51.054) (width 0.25) (layer F.Cu) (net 7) (status 20))
 (segment (start 137.90676 53.406) (end 139.634 53.406) (width 0.25) (layer B.Cu) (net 8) (status 30))
 (segment (start 139.634 53.406) (end 140.208 52.832) (width 0.25) (layer B.Cu) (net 8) (status 30))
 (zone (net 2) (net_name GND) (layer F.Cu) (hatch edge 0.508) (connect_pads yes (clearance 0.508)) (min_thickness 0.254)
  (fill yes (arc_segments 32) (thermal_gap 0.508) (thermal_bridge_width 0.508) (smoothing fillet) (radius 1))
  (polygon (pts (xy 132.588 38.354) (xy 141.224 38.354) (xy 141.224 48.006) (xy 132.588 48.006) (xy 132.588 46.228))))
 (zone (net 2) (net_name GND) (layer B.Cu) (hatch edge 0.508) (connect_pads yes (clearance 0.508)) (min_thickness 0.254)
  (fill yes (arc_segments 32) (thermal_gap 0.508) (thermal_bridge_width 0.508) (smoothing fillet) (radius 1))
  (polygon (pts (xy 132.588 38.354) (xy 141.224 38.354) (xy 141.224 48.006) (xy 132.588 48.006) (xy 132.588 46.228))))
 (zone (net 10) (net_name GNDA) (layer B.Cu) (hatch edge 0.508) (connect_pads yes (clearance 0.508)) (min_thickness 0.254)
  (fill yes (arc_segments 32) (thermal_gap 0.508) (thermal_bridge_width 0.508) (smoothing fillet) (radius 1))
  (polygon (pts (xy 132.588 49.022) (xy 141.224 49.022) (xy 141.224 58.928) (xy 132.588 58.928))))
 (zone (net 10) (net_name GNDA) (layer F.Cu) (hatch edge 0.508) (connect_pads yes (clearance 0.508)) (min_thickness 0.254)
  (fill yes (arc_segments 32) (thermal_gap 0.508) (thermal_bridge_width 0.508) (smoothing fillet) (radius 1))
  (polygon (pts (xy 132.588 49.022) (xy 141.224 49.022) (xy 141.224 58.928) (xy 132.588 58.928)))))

